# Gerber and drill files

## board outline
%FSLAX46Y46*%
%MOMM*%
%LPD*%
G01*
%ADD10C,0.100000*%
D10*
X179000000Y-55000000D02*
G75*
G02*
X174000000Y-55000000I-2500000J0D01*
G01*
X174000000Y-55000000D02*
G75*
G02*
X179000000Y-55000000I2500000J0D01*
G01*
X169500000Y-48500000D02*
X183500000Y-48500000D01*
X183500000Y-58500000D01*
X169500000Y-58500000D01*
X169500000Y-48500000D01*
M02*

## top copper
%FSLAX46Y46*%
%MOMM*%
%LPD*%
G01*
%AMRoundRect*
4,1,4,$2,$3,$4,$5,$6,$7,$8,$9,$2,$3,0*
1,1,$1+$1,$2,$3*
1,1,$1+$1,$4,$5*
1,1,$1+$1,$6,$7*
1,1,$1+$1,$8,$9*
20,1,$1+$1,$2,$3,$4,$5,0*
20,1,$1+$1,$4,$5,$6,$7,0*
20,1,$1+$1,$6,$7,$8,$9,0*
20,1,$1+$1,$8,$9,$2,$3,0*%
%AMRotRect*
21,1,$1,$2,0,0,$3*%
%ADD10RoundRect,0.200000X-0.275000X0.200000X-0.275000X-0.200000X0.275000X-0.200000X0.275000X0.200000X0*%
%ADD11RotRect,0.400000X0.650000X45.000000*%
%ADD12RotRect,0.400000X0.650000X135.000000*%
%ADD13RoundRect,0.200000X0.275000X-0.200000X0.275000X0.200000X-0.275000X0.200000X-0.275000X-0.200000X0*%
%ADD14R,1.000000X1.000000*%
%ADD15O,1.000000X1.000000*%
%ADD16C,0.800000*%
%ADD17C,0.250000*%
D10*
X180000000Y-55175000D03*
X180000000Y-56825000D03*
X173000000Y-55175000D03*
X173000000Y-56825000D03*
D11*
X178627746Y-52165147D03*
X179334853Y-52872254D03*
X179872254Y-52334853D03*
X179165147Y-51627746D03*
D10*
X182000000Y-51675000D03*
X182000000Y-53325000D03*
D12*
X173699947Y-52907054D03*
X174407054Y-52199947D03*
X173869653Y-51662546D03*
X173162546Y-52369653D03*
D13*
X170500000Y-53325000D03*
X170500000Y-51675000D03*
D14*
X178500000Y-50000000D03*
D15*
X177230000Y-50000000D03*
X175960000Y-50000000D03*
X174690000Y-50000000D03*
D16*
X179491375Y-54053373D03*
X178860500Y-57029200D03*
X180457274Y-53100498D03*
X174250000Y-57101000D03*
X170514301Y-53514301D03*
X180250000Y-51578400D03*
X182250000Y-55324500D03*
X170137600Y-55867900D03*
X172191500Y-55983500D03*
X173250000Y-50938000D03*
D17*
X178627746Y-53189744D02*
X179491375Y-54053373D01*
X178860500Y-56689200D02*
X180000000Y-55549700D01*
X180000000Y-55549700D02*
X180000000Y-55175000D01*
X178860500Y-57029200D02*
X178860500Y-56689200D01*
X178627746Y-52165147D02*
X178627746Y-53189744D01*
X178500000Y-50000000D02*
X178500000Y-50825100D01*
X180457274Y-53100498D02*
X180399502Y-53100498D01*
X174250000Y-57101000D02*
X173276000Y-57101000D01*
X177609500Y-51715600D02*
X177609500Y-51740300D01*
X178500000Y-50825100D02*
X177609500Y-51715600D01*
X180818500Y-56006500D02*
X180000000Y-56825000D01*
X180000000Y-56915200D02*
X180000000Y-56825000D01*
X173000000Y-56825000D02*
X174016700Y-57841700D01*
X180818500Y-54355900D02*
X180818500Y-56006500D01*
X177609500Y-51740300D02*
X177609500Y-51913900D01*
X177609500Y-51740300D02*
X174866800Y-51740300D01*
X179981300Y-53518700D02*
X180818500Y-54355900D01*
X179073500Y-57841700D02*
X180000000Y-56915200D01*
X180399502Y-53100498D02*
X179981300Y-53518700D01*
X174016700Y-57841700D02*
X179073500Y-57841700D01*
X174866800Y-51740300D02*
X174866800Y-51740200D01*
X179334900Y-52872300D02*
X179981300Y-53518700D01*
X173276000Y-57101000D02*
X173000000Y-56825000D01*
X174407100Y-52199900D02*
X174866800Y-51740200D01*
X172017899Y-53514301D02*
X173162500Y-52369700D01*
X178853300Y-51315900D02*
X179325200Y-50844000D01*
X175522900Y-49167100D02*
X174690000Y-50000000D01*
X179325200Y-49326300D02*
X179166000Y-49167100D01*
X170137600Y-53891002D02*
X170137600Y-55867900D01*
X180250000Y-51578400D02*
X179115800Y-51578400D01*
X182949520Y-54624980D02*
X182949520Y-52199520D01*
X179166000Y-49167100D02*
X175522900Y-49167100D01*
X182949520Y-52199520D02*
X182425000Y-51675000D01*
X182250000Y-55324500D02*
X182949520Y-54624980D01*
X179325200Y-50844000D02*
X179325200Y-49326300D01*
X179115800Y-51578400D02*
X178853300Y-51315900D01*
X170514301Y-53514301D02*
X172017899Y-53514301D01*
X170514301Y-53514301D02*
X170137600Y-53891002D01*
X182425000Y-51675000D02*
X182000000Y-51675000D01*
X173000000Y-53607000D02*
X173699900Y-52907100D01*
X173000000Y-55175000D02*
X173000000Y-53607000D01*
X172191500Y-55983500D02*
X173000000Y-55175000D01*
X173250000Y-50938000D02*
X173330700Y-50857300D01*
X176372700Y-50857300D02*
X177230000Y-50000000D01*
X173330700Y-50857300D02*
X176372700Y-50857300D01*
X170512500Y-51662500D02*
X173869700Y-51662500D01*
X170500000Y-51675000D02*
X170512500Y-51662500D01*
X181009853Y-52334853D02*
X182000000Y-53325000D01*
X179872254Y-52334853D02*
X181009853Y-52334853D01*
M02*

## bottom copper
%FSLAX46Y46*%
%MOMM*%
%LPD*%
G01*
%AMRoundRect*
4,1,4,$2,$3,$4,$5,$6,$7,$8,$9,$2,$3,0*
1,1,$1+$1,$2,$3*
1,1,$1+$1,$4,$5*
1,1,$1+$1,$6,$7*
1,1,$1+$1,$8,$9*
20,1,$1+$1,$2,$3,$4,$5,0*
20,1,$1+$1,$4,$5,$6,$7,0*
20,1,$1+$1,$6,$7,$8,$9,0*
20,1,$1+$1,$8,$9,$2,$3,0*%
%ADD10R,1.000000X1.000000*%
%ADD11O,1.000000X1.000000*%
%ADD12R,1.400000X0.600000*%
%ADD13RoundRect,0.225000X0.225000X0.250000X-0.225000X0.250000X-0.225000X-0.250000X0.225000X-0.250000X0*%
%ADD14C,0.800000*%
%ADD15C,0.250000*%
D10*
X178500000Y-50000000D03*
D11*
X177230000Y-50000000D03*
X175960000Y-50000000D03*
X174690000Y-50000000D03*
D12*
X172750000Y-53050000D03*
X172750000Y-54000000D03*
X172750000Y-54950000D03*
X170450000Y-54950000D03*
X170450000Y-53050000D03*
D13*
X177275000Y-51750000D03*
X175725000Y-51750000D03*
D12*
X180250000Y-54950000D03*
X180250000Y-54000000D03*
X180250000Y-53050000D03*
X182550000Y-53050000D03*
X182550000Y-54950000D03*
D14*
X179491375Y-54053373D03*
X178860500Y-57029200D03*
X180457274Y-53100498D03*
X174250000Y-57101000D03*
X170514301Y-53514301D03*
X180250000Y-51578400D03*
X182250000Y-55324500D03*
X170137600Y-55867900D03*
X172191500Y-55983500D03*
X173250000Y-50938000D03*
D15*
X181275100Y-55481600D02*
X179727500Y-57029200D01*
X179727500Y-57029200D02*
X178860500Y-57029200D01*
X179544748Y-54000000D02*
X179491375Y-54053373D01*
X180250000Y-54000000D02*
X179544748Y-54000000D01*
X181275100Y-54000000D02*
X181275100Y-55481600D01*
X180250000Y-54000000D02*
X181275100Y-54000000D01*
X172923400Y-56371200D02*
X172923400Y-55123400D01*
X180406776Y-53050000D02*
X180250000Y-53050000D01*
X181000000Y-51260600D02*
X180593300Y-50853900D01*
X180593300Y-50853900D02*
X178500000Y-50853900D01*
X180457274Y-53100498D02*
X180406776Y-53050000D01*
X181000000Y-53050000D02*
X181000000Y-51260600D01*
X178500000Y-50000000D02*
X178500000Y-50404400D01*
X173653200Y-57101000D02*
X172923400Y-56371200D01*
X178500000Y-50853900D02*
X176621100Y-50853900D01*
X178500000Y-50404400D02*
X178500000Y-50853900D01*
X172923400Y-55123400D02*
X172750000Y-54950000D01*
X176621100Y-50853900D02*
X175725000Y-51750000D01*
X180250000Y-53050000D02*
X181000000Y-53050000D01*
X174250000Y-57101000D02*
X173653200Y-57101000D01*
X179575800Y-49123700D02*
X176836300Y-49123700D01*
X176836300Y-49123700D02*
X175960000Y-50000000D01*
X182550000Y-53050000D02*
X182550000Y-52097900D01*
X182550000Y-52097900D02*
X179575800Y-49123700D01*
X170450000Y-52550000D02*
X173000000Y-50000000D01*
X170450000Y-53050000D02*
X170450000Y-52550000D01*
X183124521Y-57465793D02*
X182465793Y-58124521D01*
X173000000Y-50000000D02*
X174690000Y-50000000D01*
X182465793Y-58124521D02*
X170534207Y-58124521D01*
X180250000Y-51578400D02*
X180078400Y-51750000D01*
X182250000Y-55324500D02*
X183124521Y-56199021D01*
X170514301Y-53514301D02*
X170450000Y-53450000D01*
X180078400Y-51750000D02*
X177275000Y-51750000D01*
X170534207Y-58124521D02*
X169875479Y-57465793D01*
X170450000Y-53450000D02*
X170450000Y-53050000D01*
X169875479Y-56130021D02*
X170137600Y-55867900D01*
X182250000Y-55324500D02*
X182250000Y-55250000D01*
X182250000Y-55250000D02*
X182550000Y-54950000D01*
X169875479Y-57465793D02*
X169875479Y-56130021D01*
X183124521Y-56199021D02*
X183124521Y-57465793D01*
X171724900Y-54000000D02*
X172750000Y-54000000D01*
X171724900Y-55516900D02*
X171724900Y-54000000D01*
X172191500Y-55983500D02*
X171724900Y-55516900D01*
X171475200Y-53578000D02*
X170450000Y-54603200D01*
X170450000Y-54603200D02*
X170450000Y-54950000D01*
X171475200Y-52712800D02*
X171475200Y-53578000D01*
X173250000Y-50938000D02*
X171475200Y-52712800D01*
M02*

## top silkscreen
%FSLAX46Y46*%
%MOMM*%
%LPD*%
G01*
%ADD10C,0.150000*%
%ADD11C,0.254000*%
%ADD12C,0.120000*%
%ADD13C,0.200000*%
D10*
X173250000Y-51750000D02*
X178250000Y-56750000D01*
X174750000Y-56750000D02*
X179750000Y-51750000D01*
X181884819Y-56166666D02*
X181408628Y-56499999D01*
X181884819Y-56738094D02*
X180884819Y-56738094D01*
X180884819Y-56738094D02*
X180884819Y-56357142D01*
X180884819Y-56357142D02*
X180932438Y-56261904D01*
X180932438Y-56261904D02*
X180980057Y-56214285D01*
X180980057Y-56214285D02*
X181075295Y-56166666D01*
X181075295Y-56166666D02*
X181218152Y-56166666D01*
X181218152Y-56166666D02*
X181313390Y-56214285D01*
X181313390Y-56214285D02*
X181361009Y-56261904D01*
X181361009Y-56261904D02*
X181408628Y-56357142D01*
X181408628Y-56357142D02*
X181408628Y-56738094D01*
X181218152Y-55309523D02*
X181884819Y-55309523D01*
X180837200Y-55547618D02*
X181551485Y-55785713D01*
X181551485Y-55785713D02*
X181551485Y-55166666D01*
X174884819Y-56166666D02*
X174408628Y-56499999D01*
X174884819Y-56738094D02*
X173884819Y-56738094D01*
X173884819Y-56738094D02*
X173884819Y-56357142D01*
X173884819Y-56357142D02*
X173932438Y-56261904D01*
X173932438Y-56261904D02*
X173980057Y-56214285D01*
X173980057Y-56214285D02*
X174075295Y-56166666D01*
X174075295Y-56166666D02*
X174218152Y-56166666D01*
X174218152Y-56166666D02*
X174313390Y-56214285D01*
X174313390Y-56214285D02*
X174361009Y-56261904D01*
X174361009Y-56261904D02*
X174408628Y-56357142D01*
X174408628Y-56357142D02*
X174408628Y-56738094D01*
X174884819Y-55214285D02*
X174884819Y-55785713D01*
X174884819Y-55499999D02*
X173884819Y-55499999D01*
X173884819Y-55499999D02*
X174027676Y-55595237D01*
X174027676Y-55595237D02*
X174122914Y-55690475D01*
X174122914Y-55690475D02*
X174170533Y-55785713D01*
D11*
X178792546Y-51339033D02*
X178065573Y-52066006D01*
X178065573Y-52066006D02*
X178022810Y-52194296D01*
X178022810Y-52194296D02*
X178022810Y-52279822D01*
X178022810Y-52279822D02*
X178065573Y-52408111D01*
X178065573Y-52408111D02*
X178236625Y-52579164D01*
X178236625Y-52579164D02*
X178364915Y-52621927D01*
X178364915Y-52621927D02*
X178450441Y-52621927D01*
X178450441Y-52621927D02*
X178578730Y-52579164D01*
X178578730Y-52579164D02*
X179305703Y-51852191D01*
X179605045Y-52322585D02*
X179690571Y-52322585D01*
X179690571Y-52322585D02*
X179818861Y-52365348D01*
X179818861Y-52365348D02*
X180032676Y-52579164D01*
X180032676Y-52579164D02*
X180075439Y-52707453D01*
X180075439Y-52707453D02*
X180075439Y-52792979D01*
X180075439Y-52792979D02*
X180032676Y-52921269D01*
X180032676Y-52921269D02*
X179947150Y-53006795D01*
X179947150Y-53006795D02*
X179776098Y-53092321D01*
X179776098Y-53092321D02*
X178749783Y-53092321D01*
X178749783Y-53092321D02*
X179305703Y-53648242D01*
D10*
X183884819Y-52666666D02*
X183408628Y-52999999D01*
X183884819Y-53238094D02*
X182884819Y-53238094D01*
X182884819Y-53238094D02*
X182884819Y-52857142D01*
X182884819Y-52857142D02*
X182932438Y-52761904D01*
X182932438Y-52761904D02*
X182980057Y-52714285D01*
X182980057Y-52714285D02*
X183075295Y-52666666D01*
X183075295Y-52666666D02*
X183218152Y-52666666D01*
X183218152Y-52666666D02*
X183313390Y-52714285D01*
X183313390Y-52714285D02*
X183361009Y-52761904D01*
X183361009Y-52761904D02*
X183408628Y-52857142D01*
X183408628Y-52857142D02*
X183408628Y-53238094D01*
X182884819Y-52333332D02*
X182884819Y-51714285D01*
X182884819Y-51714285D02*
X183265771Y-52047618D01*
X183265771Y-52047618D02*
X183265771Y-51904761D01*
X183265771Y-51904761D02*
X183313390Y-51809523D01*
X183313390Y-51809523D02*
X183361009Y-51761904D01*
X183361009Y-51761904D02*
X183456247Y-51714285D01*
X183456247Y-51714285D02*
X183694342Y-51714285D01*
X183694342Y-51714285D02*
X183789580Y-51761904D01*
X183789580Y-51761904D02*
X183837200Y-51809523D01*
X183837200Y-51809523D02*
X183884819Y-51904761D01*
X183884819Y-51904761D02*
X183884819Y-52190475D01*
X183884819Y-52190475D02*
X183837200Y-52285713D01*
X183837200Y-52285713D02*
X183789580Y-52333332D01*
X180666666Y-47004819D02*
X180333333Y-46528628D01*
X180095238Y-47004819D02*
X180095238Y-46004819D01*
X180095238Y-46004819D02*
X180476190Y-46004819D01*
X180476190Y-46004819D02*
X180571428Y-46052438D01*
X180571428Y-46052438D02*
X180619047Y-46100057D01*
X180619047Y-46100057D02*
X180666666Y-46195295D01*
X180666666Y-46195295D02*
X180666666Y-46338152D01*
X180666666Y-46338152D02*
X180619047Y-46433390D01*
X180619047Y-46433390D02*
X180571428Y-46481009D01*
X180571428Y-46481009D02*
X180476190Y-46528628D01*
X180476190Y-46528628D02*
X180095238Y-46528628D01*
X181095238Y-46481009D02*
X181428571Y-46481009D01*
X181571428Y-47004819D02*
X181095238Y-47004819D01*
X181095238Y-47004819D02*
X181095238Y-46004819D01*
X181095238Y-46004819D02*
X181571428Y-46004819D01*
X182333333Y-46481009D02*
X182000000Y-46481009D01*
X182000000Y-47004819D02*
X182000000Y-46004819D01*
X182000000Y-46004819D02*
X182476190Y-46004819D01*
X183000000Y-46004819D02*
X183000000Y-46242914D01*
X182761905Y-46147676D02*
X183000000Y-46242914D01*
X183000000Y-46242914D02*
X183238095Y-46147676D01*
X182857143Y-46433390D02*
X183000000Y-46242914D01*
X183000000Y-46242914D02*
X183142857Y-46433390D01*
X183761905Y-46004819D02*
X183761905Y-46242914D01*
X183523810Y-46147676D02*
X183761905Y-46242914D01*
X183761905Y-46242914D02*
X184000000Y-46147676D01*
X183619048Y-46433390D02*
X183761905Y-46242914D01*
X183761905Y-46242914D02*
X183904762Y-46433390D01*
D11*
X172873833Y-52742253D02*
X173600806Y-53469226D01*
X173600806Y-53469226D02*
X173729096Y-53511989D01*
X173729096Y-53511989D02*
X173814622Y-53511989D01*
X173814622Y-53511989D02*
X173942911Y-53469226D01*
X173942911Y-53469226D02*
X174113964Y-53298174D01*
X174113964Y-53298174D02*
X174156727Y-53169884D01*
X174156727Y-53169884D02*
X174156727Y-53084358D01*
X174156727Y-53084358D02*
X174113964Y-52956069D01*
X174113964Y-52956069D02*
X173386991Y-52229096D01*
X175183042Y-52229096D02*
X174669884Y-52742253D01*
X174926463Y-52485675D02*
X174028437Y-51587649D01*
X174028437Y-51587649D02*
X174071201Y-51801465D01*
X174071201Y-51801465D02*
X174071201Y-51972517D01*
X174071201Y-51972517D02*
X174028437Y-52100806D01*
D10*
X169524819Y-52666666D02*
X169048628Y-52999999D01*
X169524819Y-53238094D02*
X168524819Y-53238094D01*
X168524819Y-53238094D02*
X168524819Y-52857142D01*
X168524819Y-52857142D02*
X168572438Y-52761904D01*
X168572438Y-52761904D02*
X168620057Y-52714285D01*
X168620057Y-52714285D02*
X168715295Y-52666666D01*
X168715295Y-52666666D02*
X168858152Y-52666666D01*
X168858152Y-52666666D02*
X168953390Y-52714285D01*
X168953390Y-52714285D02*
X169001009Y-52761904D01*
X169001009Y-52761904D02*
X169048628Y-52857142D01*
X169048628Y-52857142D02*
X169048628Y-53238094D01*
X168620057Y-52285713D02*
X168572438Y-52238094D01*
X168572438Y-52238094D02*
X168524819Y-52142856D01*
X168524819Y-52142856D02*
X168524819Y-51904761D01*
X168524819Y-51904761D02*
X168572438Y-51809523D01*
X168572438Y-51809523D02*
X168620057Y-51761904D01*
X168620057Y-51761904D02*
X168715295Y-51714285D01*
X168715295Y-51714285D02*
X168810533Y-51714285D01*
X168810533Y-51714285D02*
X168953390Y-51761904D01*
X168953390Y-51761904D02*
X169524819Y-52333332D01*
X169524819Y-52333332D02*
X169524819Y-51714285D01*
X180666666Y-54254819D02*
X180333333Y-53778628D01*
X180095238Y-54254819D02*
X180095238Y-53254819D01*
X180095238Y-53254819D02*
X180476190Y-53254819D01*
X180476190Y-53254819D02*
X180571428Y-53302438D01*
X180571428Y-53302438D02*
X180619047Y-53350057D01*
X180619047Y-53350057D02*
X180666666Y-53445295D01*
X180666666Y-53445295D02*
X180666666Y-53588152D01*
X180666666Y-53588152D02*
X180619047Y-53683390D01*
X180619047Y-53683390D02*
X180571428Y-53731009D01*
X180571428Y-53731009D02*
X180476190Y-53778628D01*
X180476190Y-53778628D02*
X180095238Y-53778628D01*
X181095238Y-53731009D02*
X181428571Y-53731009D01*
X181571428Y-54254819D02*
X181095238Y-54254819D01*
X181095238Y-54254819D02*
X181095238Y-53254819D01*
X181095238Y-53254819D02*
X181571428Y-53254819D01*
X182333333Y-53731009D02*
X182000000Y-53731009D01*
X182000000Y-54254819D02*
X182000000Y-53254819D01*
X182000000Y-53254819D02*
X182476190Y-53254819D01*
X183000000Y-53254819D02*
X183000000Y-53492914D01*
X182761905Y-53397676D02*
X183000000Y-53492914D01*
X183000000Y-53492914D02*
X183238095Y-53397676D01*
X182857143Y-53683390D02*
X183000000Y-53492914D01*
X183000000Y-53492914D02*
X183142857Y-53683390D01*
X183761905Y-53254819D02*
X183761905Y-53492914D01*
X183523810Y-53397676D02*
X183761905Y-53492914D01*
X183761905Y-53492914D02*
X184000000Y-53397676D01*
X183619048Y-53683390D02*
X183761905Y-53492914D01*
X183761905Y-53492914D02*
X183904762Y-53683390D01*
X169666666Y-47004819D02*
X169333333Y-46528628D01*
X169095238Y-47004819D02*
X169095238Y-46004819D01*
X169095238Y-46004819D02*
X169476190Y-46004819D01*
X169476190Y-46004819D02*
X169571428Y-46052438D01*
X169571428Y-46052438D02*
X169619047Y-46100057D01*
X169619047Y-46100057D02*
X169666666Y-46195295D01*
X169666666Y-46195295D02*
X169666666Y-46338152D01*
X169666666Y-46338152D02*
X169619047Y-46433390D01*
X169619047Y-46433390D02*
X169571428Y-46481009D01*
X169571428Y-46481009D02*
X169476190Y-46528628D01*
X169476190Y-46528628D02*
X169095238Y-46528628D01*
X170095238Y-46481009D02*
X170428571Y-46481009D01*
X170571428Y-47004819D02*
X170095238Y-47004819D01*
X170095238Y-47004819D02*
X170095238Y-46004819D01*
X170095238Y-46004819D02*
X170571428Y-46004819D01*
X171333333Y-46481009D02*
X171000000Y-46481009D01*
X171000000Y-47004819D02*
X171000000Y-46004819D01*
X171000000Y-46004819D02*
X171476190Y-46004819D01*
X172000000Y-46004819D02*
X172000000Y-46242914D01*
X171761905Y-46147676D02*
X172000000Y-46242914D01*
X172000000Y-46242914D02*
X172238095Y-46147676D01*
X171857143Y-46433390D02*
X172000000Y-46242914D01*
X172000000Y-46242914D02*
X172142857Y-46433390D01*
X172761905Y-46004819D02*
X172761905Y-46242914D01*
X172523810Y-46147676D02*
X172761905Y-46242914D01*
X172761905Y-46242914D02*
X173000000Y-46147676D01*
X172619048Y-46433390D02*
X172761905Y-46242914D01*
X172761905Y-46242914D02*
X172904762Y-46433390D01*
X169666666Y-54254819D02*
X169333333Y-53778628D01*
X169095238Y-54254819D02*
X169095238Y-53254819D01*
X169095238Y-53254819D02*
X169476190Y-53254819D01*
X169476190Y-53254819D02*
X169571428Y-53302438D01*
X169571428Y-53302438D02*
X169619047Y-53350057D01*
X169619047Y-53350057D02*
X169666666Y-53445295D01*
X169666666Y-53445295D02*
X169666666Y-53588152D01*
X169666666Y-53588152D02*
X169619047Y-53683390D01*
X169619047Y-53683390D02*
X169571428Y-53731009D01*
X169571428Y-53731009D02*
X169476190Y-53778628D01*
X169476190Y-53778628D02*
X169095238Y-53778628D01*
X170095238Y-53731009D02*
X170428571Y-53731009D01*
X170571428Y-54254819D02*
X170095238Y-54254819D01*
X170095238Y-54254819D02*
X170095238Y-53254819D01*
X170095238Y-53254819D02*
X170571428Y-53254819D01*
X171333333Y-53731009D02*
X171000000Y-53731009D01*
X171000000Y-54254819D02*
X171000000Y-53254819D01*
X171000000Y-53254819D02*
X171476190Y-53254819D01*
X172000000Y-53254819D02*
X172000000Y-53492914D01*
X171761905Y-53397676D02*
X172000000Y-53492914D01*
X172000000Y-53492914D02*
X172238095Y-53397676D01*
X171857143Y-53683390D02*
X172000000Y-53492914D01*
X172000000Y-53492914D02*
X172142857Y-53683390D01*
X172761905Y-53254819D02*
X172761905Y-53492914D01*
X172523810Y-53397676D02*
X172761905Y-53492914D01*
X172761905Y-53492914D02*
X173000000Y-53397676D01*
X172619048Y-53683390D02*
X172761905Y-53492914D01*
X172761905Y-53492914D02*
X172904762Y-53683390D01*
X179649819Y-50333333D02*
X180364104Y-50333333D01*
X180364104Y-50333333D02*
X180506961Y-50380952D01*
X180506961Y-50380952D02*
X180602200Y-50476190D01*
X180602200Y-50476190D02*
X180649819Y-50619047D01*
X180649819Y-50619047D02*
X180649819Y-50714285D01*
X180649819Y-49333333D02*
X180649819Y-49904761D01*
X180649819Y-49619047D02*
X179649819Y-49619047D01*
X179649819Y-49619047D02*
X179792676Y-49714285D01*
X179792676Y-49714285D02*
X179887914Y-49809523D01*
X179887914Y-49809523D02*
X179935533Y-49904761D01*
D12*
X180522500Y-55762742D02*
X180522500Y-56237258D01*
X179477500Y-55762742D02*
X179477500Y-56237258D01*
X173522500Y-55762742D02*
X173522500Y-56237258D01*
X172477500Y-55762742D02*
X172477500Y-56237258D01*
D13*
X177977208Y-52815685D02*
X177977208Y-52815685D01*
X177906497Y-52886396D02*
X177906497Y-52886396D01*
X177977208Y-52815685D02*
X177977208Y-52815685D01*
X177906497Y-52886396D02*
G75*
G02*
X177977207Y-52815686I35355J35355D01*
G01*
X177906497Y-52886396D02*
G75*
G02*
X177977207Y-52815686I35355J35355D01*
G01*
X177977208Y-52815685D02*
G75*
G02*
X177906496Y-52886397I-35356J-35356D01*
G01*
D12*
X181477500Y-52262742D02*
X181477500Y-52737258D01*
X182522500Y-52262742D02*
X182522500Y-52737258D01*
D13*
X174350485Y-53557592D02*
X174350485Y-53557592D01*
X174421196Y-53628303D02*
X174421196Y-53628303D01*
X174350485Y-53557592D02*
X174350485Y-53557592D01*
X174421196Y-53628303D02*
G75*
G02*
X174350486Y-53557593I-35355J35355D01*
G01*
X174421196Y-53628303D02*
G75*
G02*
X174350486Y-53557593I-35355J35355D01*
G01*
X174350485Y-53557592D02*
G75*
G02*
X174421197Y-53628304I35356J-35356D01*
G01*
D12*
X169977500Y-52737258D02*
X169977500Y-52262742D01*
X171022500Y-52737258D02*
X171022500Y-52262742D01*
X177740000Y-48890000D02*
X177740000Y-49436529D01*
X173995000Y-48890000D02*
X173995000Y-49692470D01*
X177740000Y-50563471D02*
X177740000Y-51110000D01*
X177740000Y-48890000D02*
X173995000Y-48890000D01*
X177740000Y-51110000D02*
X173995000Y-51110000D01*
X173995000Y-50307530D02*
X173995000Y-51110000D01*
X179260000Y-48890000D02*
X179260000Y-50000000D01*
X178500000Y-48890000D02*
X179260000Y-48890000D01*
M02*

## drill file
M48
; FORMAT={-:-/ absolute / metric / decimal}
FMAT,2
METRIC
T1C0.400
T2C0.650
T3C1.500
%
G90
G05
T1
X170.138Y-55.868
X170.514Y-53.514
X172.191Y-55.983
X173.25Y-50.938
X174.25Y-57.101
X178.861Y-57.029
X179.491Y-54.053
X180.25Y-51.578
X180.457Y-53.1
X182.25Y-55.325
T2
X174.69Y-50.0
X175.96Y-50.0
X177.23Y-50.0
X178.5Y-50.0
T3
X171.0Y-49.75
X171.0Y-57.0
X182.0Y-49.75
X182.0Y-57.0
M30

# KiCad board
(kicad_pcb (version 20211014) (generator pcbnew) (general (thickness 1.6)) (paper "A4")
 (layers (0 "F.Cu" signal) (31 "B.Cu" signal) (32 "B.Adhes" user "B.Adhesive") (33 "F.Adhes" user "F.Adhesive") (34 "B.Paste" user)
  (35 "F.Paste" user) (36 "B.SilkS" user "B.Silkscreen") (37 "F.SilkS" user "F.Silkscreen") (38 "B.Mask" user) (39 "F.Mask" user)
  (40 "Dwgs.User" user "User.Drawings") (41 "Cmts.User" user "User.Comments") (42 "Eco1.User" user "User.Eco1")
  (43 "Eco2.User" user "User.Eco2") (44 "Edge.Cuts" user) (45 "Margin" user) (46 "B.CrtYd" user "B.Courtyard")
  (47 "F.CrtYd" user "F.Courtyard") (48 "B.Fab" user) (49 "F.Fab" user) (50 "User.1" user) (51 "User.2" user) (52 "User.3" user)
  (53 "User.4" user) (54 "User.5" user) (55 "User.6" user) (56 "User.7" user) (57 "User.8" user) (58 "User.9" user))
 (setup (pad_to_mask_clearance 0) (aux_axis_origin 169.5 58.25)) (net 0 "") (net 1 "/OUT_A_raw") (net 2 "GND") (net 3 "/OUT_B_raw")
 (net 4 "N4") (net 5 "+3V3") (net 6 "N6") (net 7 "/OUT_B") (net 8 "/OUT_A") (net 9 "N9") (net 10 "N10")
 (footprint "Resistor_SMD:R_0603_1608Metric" (layer "F.Cu") (at 180 56 -90)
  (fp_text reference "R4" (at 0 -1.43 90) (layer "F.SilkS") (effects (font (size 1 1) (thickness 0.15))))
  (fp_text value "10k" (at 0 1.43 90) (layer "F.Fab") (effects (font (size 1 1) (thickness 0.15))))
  (fp_line (start -0.237258 -0.5225) (end 0.237258 -0.5225) (layer "F.SilkS") (width 0.12))
  (fp_line (start -0.237258 0.5225) (end 0.237258 0.5225) (layer "F.SilkS") (width 0.12))
  (pad "1" smd roundrect (at -0.825 0 270) (size 0.8 0.95) (layers "F.Cu" "F.Paste" "F.Mask") (roundrect_rratio 0.25) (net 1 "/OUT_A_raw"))
  (pad "2" smd roundrect (at 0.825 0 270) (size 0.8 0.95) (layers "F.Cu" "F.Paste" "F.Mask") (roundrect_rratio 0.25) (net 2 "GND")))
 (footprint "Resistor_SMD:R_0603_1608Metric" (layer "F.Cu") (at 173 56 -90)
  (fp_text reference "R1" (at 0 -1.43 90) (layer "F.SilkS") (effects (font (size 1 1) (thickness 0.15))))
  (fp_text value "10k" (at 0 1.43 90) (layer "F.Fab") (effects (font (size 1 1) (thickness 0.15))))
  (fp_line (start -0.237258 -0.5225) (end 0.237258 -0.5225) (layer "F.SilkS") (width 0.12))
  (fp_line (start -0.237258 0.5225) (end 0.237258 0.5225) (layer "F.SilkS") (width 0.12))
  (pad "1" smd roundrect (at -0.825 0 270) (size 0.8 0.95) (layers "F.Cu" "F.Paste" "F.Mask") (roundrect_rratio 0.25) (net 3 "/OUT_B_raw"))
  (pad "2" smd roundrect (at 0.825 0 270) (size 0.8 0.95) (layers "F.Cu" "F.Paste" "F.Mask") (roundrect_rratio 0.25) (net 2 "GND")))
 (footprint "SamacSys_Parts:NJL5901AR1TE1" (layer "F.Cu") (at 179.25 52.25 -45)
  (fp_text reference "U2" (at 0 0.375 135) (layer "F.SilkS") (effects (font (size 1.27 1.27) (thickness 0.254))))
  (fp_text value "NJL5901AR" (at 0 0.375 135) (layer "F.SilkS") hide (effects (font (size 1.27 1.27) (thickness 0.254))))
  (fp_line (start -0.5 1.3) (end -0.5 1.3) (layer "F.SilkS") (width 0.2))
  (fp_line (start -0.5 1.4) (end -0.5 1.4) (layer "F.SilkS") (width 0.2))
  (fp_line (start -0.5 1.3) (end -0.5 1.3) (layer "F.SilkS") (width 0.2))
  (fp_arc (start -0.5 1.4) (mid -0.55 1.35) (end -0.5 1.3) (layer "F.SilkS") (width 0.2))
  (fp_arc (start -0.5 1.4) (mid -0.55 1.35) (end -0.5 1.3) (layer "F.SilkS") (width 0.2))
  (fp_arc (start -0.5 1.3) (mid -0.45 1.35) (end -0.5 1.4) (layer "F.SilkS") (width 0.2))
  (pad "1" smd rect locked (at -0.5 0.38 45) (size 0.4 0.65) (layers "F.Cu" "F.Paste" "F.Mask") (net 1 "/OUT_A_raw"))
  (pad "2" smd rect locked (at 0.5 0.38 45) (size 0.4 0.65) (layers "F.Cu" "F.Paste" "F.Mask") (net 2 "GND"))
  (pad "3" smd rect locked (at 0.5 -0.38 45) (size 0.4 0.65) (layers "F.Cu" "F.Paste" "F.Mask") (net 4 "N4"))
  (pad "4" smd rect locked (at -0.5 -0.38 45) (size 0.4 0.65) (layers "F.Cu" "F.Paste" "F.Mask") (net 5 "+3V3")))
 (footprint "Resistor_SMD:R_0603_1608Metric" (layer "F.Cu") (at 182 52.5 -90)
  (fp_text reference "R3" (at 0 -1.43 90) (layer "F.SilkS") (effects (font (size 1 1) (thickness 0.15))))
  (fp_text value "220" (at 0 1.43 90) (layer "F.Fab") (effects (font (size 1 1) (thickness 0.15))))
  (fp_line (start -0.237258 0.5225) (end 0.237258 0.5225) (layer "F.SilkS") (width 0.12))
  (fp_line (start -0.237258 -0.5225) (end 0.237258 -0.5225) (layer "F.SilkS") (width 0.12))
  (pad "1" smd roundrect (at -0.825 0 270) (size 0.8 0.95) (layers "F.Cu" "F.Paste" "F.Mask") (roundrect_rratio 0.25) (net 5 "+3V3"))
  (pad "2" smd roundrect (at 0.825 0 270) (size 0.8 0.95) (layers "F.Cu" "F.Paste" "F.Mask") (roundrect_rratio 0.25) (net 4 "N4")))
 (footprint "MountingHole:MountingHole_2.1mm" (layer "F.Cu") (at 182 49.75)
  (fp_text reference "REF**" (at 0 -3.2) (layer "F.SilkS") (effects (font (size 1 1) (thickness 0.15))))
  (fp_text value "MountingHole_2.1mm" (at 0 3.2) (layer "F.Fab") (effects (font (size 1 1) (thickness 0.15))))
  (pad "" np_thru_hole circle (at 0 0) (size 1.5 1.5) (drill 1.5) (layers F&B.Cu *.Mask)))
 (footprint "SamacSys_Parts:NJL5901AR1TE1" (layer "F.Cu") (at 173.7848 52.2848 45)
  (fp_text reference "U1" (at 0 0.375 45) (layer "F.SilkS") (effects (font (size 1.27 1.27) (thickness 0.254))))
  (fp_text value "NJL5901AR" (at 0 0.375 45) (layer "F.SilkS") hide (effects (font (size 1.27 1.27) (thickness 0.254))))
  (fp_line (start -0.5 1.3) (end -0.5 1.3) (layer "F.SilkS") (width 0.2))
  (fp_line (start -0.5 1.4) (end -0.5 1.4) (layer "F.SilkS") (width 0.2))
  (fp_line (start -0.5 1.3) (end -0.5 1.3) (layer "F.SilkS") (width 0.2))
  (fp_arc (start -0.5 1.4) (mid -0.55 1.35) (end -0.5 1.3) (layer "F.SilkS") (width 0.2))
  (fp_arc (start -0.5 1.4) (mid -0.55 1.35) (end -0.5 1.3) (layer "F.SilkS") (width 0.2))
  (fp_arc (start -0.5 1.3) (mid -0.45 1.35) (end -0.5 1.4) (layer "F.SilkS") (width 0.2))
  (pad "1" smd rect locked (at -0.5 0.38 135) (size 0.4 0.65) (layers "F.Cu" "F.Paste" "F.Mask") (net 3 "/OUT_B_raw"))
  (pad "2" smd rect locked (at 0.5 0.38 135) (size 0.4 0.65) (layers "F.Cu" "F.Paste" "F.Mask") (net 2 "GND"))
  (pad "3" smd rect locked (at 0.5 -0.38 135) (size 0.4 0.65) (layers "F.Cu" "F.Paste" "F.Mask") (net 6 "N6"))
  (pad "4" smd rect locked (at -0.5 -0.38 135) (size 0.4 0.65) (layers "F.Cu" "F.Paste" "F.Mask") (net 5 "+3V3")))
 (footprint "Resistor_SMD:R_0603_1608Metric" (layer "F.Cu") (at 170.5 52.5 90)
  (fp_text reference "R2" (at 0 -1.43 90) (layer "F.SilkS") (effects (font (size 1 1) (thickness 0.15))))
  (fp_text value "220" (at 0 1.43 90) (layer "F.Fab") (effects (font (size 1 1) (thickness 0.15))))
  (fp_line (start -0.237258 -0.5225) (end 0.237258 -0.5225) (layer "F.SilkS") (width 0.12))
  (fp_line (start -0.237258 0.5225) (end 0.237258 0.5225) (layer "F.SilkS") (width 0.12))
  (pad "1" smd roundrect (at -0.825 0 90) (size 0.8 0.95) (layers "F.Cu" "F.Paste" "F.Mask") (roundrect_rratio 0.25) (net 5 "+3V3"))
  (pad "2" smd roundrect (at 0.825 0 90) (size 0.8 0.95) (layers "F.Cu" "F.Paste" "F.Mask") (roundrect_rratio 0.25) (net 6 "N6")))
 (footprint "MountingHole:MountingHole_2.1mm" (layer "F.Cu") (at 182 57)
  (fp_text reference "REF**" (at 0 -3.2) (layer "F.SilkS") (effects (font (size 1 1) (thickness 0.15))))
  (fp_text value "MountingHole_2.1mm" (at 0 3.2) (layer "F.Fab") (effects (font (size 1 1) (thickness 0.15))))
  (pad "" np_thru_hole circle (at 0 0) (size 1.5 1.5) (drill 1.5) (layers F&B.Cu *.Mask)))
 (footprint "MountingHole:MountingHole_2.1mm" (layer "F.Cu") (at 171 49.75)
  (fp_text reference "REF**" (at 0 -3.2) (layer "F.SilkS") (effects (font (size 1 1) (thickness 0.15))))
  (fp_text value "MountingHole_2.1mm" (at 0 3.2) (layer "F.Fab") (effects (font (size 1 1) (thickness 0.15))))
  (pad "" np_thru_hole circle (at 0 0) (size 1.5 1.5) (drill 1.5) (layers F&B.Cu *.Mask)))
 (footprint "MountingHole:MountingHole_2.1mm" (layer "F.Cu") (at 171 57)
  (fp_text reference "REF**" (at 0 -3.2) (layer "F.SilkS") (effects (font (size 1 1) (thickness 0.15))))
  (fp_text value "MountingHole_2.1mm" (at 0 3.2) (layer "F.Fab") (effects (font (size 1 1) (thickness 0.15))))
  (pad "" np_thru_hole circle (at 0 0) (size 1.5 1.5) (drill 1.5) (layers F&B.Cu *.Mask)))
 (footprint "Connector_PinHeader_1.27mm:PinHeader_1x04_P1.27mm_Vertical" (layer "F.Cu") (at 178.5 50 -90)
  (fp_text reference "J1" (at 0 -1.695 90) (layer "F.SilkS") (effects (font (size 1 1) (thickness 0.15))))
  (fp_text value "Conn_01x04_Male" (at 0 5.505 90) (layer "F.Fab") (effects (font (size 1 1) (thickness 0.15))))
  (fp_line (start -1.11 0.76) (end -0.563471 0.76) (layer "F.SilkS") (width 0.12))
  (fp_line (start -1.11 4.505) (end -0.30753 4.505) (layer "F.SilkS") (width 0.12))
  (fp_line (start 0.563471 0.76) (end 1.11 0.76) (layer "F.SilkS") (width 0.12))
  (fp_line (start -1.11 0.76) (end -1.11 4.505) (layer "F.SilkS") (width 0.12))
  (fp_line (start 1.11 0.76) (end 1.11 4.505) (layer "F.SilkS") (width 0.12))
  (fp_line (start 0.30753 4.505) (end 1.11 4.505) (layer "F.SilkS") (width 0.12))
  (fp_line (start -1.11 -0.76) (end 0 -0.76) (layer "F.SilkS") (width 0.12))
  (fp_line (start -1.11 0) (end -1.11 -0.76) (layer "F.SilkS") (width 0.12))
  (pad "1" thru_hole rect (at 0 0 270) (size 1 1) (drill 0.65) (layers *.Cu *.Mask) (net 2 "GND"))
  (pad "2" thru_hole oval (at 0 1.27 270) (size 1 1) (drill 0.65) (layers *.Cu *.Mask) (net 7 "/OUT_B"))
  (pad "3" thru_hole oval (at 0 2.54 270) (size 1 1) (drill 0.65) (layers *.Cu *.Mask) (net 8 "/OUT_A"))
  (pad "4" thru_hole oval (at 0 3.81 270) (size 1 1) (drill 0.65) (layers *.Cu *.Mask) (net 5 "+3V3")))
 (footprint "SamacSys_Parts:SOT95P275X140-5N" (layer "B.Cu") (at 171.6 54 180)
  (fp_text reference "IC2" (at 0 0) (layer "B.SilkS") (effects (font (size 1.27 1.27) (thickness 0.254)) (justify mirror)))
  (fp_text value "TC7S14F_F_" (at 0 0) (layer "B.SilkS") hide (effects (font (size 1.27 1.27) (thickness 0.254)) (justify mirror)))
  (pad "1" smd rect locked (at -1.15 0.95 90) (size 0.6 1.4) (layers "B.Cu" "B.Paste" "B.Mask") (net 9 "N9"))
  (pad "2" smd rect locked (at -1.15 0 90) (size 0.6 1.4) (layers "B.Cu" "B.Paste" "B.Mask") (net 3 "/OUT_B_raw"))
  (pad "3" smd rect locked (at -1.15 -0.95 90) (size 0.6 1.4) (layers "B.Cu" "B.Paste" "B.Mask") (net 2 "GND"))
  (pad "4" smd rect locked (at 1.15 -0.95 90) (size 0.6 1.4) (layers "B.Cu" "B.Paste" "B.Mask") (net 7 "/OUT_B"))
  (pad "5" smd rect locked (at 1.15 0.95 90) (size 0.6 1.4) (layers "B.Cu" "B.Paste" "B.Mask") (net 5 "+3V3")))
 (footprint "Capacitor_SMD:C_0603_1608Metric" (layer "B.Cu") (at 176.5 51.75 180)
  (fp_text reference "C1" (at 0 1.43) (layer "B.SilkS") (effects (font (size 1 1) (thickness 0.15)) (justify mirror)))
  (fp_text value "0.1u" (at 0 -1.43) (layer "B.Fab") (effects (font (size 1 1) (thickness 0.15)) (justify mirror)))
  (pad "1" smd roundrect (at -0.775 0 180) (size 0.9 0.95) (layers "B.Cu" "B.Paste" "B.Mask") (roundrect_rratio 0.25) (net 5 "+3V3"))
  (pad "2" smd roundrect (at 0.775 0 180) (size 0.9 0.95) (layers "B.Cu" "B.Paste" "B.Mask") (roundrect_rratio 0.25) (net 2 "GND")))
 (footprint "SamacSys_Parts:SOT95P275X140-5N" (layer "B.Cu") (at 181.4 54)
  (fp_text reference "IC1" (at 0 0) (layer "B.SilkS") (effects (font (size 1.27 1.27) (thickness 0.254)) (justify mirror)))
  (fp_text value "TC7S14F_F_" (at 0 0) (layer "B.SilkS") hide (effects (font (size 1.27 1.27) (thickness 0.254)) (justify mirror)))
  (pad "1" smd rect locked (at -1.15 0.95 270) (size 0.6 1.4) (layers "B.Cu" "B.Paste" "B.Mask") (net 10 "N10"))
  (pad "2" smd rect locked (at -1.15 0 270) (size 0.6 1.4) (layers "B.Cu" "B.Paste" "B.Mask") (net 1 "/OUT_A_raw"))
  (pad "3" smd rect locked (at -1.15 -0.95 270) (size 0.6 1.4) (layers "B.Cu" "B.Paste" "B.Mask") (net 2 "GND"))
  (pad "4" smd rect locked (at 1.15 -0.95 270) (size 0.6 1.4) (layers "B.Cu" "B.Paste" "B.Mask") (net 8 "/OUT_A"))
  (pad "5" smd rect locked (at 1.15 0.95 270) (size 0.6 1.4) (layers "B.Cu" "B.Paste" "B.Mask") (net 5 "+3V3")))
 (gr_line (start 173.25 51.75) (end 178.25 56.75) (layer "F.SilkS") (width 0.15))
 (gr_line (start 174.75 56.75) (end 179.75 51.75) (layer "F.SilkS") (width 0.15))
 (gr_circle (center 176.5 55) (end 179 55) (layer "Edge.Cuts") (width 0.1) (fill none))
 (gr_rect (start 169.5 48.5) (end 183.5 58.5) (layer "Edge.Cuts") (width 0.1) (fill none))
 (segment (start 178.627746 53.189744) (end 179.491375 54.053373) (width 0.25) (layer "F.Cu") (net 1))
 (segment (start 178.8605 56.6892) (end 180 55.5497) (width 0.25) (layer "F.Cu") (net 1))
 (segment (start 180 55.5497) (end 180 55.175) (width 0.25) (layer "F.Cu") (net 1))
 (segment (start 178.8605 57.0292) (end 178.8605 56.6892) (width 0.25) (layer "F.Cu") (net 1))
 (segment (start 178.627746 52.165147) (end 178.627746 53.189744) (width 0.25) (layer "F.Cu") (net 1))
 (via (at 179.491375 54.053373) (size 0.8) (drill 0.4) (layers "F.Cu" "B.Cu") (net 1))
 (via (at 178.8605 57.0292) (size 0.8) (drill 0.4) (layers "F.Cu" "B.Cu") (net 1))
 (segment (start 181.2751 55.4816) (end 179.7275 57.0292) (width 0.25) (layer "B.Cu") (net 1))
 (segment (start 179.7275 57.0292) (end 178.8605 57.0292) (width 0.25) (layer "B.Cu") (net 1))
 (segment (start 179.544748 54) (end 179.491375 54.053373) (width 0.25) (layer "B.Cu") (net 1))
 (segment (start 180.25 54) (end 179.544748 54) (width 0.25) (layer "B.Cu") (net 1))
 (segment (start 181.2751 54) (end 181.2751 55.4816) (width 0.25) (layer "B.Cu") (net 1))
 (segment (start 180.25 54) (end 181.2751 54) (width 0.25) (layer "B.Cu") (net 1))
 (segment (start 178.5 50) (end 178.5 50.8251) (width 0.25) (layer "F.Cu") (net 2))
 (segment (start 180.457274 53.100498) (end 180.399502 53.100498) (width 0.25) (layer "F.Cu") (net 2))
 (segment (start 174.25 57.101) (end 173.276 57.101) (width 0.25) (layer "F.Cu") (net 2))
 (segment (start 177.6095 51.7156) (end 177.6095 51.7403) (width 0.25) (layer "F.Cu") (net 2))
 (segment (start 178.5 50.8251) (end 177.6095 51.7156) (width 0.25) (layer "F.Cu") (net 2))
 (segment (start 180.8185 56.0065) (end 180 56.825) (width 0.25) (layer "F.Cu") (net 2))
 (segment (start 180 56.9152) (end 180 56.825) (width 0.25) (layer "F.Cu") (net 2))
 (segment (start 173 56.825) (end 174.0167 57.8417) (width 0.25) (layer "F.Cu") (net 2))
 (segment (start 180.8185 54.3559) (end 180.8185 56.0065) (width 0.25) (layer "F.Cu") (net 2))
 (segment (start 177.6095 51.7403) (end 177.6095 51.9139) (width 0.25) (layer "F.Cu") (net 2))
 (segment (start 177.6095 51.7403) (end 174.8668 51.7403) (width 0.25) (layer "F.Cu") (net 2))
 (segment (start 179.9813 53.5187) (end 180.8185 54.3559) (width 0.25) (layer "F.Cu") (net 2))
 (segment (start 179.0735 57.8417) (end 180 56.9152) (width 0.25) (layer "F.Cu") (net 2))
 (segment (start 180.399502 53.100498) (end 179.9813 53.5187) (width 0.25) (layer "F.Cu") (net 2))
 (segment (start 174.0167 57.8417) (end 179.0735 57.8417) (width 0.25) (layer "F.Cu") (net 2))
 (segment (start 174.8668 51.7403) (end 174.8668 51.7402) (width 0.25) (layer "F.Cu") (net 2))
 (segment (start 179.3349 52.8723) (end 179.9813 53.5187) (width 0.25) (layer "F.Cu") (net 2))
 (segment (start 173.276 57.101) (end 173 56.825) (width 0.25) (layer "F.Cu") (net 2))
 (segment (start 174.4071 52.1999) (end 174.8668 51.7402) (width 0.25) (layer "F.Cu") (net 2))
 (via (at 180.457274 53.100498) (size 0.8) (drill 0.4) (layers "F.Cu" "B.Cu") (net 2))
 (via (at 174.25 57.101) (size 0.8) (drill 0.4) (layers "F.Cu" "B.Cu") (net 2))
 (segment (start 172.9234 56.3712) (end 172.9234 55.1234) (width 0.25) (layer "B.Cu") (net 2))
 (segment (start 180.406776 53.05) (end 180.25 53.05) (width 0.25) (layer "B.Cu") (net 2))
 (segment (start 181 51.2606) (end 180.5933 50.8539) (width 0.25) (layer "B.Cu") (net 2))
 (segment (start 180.5933 50.8539) (end 178.5 50.8539) (width 0.25) (layer "B.Cu") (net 2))
 (segment (start 180.457274 53.100498) (end 180.406776 53.05) (width 0.25) (layer "B.Cu") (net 2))
 (segment (start 181 53.05) (end 181 51.2606) (width 0.25) (layer "B.Cu") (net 2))
 (segment (start 178.5 50) (end 178.5 50.4044) (width 0.25) (layer "B.Cu") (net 2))
 (segment (start 173.6532 57.101) (end 172.9234 56.3712) (width 0.25) (layer "B.Cu") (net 2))
 (segment (start 178.5 50.8539) (end 176.6211 50.8539) (width 0.25) (layer "B.Cu") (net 2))
 (segment (start 178.5 50.4044) (end 178.5 50.8539) (width 0.25) (layer "B.Cu") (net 2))
 (segment (start 172.9234 55.1234) (end 172.75 54.95) (width 0.25) (layer "B.Cu") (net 2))
 (segment (start 176.6211 50.8539) (end 175.725 51.75) (width 0.25) (layer "B.Cu") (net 2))
 (segment (start 180.25 53.05) (end 181 53.05) (width 0.25) (layer "B.Cu") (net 2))
 (segment (start 174.25 57.101) (end 173.6532 57.101) (width 0.25) (layer "B.Cu") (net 2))
 (segment (start 179.5758 49.1237) (end 176.8363 49.1237) (width 0.25) (layer "B.Cu") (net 8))
 (segment (start 176.8363 49.1237) (end 175.96 50) (width 0.25) (layer "B.Cu") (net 8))
 (segment (start 182.55 53.05) (end 182.55 52.0979) (width 0.25) (layer "B.Cu") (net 8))
 (segment (start 182.55 52.0979) (end 179.5758 49.1237) (width 0.25) (layer "B.Cu") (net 8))
 (segment (start 172.017899 53.514301) (end 173.1625 52.3697) (width 0.25) (layer "F.Cu") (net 5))
 (segment (start 178.8533 51.3159) (end 179.3252 50.844) (width 0.25) (layer "F.Cu") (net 5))
 (segment (start 175.5229 49.1671) (end 174.69 50) (width 0.25) (layer "F.Cu") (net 5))
 (segment (start 179.3252 49.3263) (end 179.166 49.1671) (width 0.25) (layer "F.Cu") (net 5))
 (segment (start 170.1376 53.891002) (end 170.1376 55.8679) (width 0.25) (layer "F.Cu") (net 5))
 (segment (start 180.25 51.5784) (end 179.1158 51.5784) (width 0.25) (layer "F.Cu") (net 5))
 (segment (start 182.94952 54.62498) (end 182.94952 52.19952) (width 0.25) (layer "F.Cu") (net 5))
 (segment (start 179.166 49.1671) (end 175.5229 49.1671) (width 0.25) (layer "F.Cu") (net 5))
 (segment (start 182.94952 52.19952) (end 182.425 51.675) (width 0.25) (layer "F.Cu") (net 5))
 (segment (start 182.25 55.3245) (end 182.94952 54.62498) (width 0.25) (layer "F.Cu") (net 5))
 (segment (start 179.3252 50.844) (end 179.3252 49.3263) (width 0.25) (layer "F.Cu") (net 5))
 (segment (start 179.1158 51.5784) (end 178.8533 51.3159) (width 0.25) (layer "F.Cu") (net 5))
 (segment (start 170.514301 53.514301) (end 172.017899 53.514301) (width 0.25) (layer "F.Cu") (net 5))
 (segment (start 170.514301 53.514301) (end 170.1376 53.891002) (width 0.25) (layer "F.Cu") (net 5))
 (segment (start 182.425 51.675) (end 182 51.675) (width 0.25) (layer "F.Cu") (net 5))
 (via (at 170.514301 53.514301) (size 0.8) (drill 0.4) (layers "F.Cu" "B.Cu") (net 5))
 (via (at 180.25 51.5784) (size 0.8) (drill 0.4) (layers "F.Cu" "B.Cu") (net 5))
 (via (at 182.25 55.3245) (size 0.8) (drill 0.4) (layers "F.Cu" "B.Cu") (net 5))
 (via (at 170.1376 55.8679) (size 0.8) (drill 0.4) (layers "F.Cu" "B.Cu") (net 5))
 (segment (start 170.45 52.55) (end 173 50) (width 0.25) (layer "B.Cu") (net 5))
 (segment (start 170.45 53.05) (end 170.45 52.55) (width 0.25) (layer "B.Cu") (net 5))
 (segment (start 183.124521 57.465793) (end 182.465793 58.124521) (width 0.25) (layer "B.Cu") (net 5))
 (segment (start 173 50) (end 174.69 50) (width 0.25) (layer "B.Cu") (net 5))
 (segment (start 182.465793 58.124521) (end 170.534207 58.124521) (width 0.25) (layer "B.Cu") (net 5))
 (segment (start 180.25 51.5784) (end 180.0784 51.75) (width 0.25) (layer "B.Cu") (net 5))
 (segment (start 182.25 55.3245) (end 183.124521 56.199021) (width 0.25) (layer "B.Cu") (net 5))
 (segment (start 170.514301 53.514301) (end 170.45 53.45) (width 0.25) (layer "B.Cu") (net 5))
 (segment (start 180.0784 51.75) (end 177.275 51.75) (width 0.25) (layer "B.Cu") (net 5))
 (segment (start 170.534207 58.124521) (end 169.875479 57.465793) (width 0.25) (layer "B.Cu") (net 5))
 (segment (start 170.45 53.45) (end 170.45 53.05) (width 0.25) (layer "B.Cu") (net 5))
 (segment (start 169.875479 56.130021) (end 170.1376 55.8679) (width 0.25) (layer "B.Cu") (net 5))
 (segment (start 182.25 55.3245) (end 182.25 55.25) (width 0.25) (layer "B.Cu") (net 5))
 (segment (start 182.25 55.25) (end 182.55 54.95) (width 0.25) (layer "B.Cu") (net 5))
 (segment (start 169.875479 57.465793) (end 169.875479 56.130021) (width 0.25) (layer "B.Cu") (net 5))
 (segment (start 183.124521 56.199021) (end 183.124521 57.465793) (width 0.25) (layer "B.Cu") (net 5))
 (segment (start 173 53.607) (end 173.6999 52.9071) (width 0.25) (layer "F.Cu") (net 3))
 (segment (start 173 55.175) (end 173 53.607) (width 0.25) (layer "F.Cu") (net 3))
 (segment (start 172.1915 55.9835) (end 173 55.175) (width 0.25) (layer "F.Cu") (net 3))
 (via (at 172.1915 55.9835) (size 0.8) (drill 0.4) (layers "F.Cu" "B.Cu") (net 3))
 (segment (start 171.7249 54) (end 172.75 54) (width 0.25) (layer "B.Cu") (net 3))
 (segment (start 171.7249 55.5169) (end 171.7249 54) (width 0.25) (layer "B.Cu") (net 3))
 (segment (start 172.1915 55.9835) (end 171.7249 55.5169) (width 0.25) (layer "B.Cu") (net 3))
 (segment (start 173.25 50.938) (end 173.3307 50.8573) (width 0.25) (layer "F.Cu") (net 7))
 (segment (start 176.3727 50.8573) (end 177.23 50) (width 0.25) (layer "F.Cu") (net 7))
 (segment (start 173.3307 50.8573) (end 176.3727 50.8573) (width 0.25) (layer "F.Cu") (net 7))
 (via (at 173.25 50.938) (size 0.8) (drill 0.4) (layers "F.Cu" "B.Cu") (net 7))
 (segment (start 171.4752 53.578) (end 170.45 54.6032) (width 0.25) (layer "B.Cu") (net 7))
 (segment (start 170.45 54.6032) (end 170.45 54.95) (width 0.25) (layer "B.Cu") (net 7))
 (segment (start 171.4752 52.7128) (end 171.4752 53.578) (width 0.25) (layer "B.Cu") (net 7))
 (segment (start 173.25 50.938) (end 171.4752 52.7128) (width 0.25) (layer "B.Cu") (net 7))
 (segment (start 170.5125 51.6625) (end 173.8697 51.6625) (width 0.25) (layer "F.Cu") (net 6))
 (segment (start 170.5 51.675) (end 170.5125 51.6625) (width 0.25) (layer "F.Cu") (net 6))
 (segment (start 181.009853 52.334853) (end 182 53.325) (width 0.25) (layer "F.Cu") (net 4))
 (segment (start 179.872254 52.334853) (end 181.009853 52.334853) (width 0.25) (layer "F.Cu") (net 4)))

